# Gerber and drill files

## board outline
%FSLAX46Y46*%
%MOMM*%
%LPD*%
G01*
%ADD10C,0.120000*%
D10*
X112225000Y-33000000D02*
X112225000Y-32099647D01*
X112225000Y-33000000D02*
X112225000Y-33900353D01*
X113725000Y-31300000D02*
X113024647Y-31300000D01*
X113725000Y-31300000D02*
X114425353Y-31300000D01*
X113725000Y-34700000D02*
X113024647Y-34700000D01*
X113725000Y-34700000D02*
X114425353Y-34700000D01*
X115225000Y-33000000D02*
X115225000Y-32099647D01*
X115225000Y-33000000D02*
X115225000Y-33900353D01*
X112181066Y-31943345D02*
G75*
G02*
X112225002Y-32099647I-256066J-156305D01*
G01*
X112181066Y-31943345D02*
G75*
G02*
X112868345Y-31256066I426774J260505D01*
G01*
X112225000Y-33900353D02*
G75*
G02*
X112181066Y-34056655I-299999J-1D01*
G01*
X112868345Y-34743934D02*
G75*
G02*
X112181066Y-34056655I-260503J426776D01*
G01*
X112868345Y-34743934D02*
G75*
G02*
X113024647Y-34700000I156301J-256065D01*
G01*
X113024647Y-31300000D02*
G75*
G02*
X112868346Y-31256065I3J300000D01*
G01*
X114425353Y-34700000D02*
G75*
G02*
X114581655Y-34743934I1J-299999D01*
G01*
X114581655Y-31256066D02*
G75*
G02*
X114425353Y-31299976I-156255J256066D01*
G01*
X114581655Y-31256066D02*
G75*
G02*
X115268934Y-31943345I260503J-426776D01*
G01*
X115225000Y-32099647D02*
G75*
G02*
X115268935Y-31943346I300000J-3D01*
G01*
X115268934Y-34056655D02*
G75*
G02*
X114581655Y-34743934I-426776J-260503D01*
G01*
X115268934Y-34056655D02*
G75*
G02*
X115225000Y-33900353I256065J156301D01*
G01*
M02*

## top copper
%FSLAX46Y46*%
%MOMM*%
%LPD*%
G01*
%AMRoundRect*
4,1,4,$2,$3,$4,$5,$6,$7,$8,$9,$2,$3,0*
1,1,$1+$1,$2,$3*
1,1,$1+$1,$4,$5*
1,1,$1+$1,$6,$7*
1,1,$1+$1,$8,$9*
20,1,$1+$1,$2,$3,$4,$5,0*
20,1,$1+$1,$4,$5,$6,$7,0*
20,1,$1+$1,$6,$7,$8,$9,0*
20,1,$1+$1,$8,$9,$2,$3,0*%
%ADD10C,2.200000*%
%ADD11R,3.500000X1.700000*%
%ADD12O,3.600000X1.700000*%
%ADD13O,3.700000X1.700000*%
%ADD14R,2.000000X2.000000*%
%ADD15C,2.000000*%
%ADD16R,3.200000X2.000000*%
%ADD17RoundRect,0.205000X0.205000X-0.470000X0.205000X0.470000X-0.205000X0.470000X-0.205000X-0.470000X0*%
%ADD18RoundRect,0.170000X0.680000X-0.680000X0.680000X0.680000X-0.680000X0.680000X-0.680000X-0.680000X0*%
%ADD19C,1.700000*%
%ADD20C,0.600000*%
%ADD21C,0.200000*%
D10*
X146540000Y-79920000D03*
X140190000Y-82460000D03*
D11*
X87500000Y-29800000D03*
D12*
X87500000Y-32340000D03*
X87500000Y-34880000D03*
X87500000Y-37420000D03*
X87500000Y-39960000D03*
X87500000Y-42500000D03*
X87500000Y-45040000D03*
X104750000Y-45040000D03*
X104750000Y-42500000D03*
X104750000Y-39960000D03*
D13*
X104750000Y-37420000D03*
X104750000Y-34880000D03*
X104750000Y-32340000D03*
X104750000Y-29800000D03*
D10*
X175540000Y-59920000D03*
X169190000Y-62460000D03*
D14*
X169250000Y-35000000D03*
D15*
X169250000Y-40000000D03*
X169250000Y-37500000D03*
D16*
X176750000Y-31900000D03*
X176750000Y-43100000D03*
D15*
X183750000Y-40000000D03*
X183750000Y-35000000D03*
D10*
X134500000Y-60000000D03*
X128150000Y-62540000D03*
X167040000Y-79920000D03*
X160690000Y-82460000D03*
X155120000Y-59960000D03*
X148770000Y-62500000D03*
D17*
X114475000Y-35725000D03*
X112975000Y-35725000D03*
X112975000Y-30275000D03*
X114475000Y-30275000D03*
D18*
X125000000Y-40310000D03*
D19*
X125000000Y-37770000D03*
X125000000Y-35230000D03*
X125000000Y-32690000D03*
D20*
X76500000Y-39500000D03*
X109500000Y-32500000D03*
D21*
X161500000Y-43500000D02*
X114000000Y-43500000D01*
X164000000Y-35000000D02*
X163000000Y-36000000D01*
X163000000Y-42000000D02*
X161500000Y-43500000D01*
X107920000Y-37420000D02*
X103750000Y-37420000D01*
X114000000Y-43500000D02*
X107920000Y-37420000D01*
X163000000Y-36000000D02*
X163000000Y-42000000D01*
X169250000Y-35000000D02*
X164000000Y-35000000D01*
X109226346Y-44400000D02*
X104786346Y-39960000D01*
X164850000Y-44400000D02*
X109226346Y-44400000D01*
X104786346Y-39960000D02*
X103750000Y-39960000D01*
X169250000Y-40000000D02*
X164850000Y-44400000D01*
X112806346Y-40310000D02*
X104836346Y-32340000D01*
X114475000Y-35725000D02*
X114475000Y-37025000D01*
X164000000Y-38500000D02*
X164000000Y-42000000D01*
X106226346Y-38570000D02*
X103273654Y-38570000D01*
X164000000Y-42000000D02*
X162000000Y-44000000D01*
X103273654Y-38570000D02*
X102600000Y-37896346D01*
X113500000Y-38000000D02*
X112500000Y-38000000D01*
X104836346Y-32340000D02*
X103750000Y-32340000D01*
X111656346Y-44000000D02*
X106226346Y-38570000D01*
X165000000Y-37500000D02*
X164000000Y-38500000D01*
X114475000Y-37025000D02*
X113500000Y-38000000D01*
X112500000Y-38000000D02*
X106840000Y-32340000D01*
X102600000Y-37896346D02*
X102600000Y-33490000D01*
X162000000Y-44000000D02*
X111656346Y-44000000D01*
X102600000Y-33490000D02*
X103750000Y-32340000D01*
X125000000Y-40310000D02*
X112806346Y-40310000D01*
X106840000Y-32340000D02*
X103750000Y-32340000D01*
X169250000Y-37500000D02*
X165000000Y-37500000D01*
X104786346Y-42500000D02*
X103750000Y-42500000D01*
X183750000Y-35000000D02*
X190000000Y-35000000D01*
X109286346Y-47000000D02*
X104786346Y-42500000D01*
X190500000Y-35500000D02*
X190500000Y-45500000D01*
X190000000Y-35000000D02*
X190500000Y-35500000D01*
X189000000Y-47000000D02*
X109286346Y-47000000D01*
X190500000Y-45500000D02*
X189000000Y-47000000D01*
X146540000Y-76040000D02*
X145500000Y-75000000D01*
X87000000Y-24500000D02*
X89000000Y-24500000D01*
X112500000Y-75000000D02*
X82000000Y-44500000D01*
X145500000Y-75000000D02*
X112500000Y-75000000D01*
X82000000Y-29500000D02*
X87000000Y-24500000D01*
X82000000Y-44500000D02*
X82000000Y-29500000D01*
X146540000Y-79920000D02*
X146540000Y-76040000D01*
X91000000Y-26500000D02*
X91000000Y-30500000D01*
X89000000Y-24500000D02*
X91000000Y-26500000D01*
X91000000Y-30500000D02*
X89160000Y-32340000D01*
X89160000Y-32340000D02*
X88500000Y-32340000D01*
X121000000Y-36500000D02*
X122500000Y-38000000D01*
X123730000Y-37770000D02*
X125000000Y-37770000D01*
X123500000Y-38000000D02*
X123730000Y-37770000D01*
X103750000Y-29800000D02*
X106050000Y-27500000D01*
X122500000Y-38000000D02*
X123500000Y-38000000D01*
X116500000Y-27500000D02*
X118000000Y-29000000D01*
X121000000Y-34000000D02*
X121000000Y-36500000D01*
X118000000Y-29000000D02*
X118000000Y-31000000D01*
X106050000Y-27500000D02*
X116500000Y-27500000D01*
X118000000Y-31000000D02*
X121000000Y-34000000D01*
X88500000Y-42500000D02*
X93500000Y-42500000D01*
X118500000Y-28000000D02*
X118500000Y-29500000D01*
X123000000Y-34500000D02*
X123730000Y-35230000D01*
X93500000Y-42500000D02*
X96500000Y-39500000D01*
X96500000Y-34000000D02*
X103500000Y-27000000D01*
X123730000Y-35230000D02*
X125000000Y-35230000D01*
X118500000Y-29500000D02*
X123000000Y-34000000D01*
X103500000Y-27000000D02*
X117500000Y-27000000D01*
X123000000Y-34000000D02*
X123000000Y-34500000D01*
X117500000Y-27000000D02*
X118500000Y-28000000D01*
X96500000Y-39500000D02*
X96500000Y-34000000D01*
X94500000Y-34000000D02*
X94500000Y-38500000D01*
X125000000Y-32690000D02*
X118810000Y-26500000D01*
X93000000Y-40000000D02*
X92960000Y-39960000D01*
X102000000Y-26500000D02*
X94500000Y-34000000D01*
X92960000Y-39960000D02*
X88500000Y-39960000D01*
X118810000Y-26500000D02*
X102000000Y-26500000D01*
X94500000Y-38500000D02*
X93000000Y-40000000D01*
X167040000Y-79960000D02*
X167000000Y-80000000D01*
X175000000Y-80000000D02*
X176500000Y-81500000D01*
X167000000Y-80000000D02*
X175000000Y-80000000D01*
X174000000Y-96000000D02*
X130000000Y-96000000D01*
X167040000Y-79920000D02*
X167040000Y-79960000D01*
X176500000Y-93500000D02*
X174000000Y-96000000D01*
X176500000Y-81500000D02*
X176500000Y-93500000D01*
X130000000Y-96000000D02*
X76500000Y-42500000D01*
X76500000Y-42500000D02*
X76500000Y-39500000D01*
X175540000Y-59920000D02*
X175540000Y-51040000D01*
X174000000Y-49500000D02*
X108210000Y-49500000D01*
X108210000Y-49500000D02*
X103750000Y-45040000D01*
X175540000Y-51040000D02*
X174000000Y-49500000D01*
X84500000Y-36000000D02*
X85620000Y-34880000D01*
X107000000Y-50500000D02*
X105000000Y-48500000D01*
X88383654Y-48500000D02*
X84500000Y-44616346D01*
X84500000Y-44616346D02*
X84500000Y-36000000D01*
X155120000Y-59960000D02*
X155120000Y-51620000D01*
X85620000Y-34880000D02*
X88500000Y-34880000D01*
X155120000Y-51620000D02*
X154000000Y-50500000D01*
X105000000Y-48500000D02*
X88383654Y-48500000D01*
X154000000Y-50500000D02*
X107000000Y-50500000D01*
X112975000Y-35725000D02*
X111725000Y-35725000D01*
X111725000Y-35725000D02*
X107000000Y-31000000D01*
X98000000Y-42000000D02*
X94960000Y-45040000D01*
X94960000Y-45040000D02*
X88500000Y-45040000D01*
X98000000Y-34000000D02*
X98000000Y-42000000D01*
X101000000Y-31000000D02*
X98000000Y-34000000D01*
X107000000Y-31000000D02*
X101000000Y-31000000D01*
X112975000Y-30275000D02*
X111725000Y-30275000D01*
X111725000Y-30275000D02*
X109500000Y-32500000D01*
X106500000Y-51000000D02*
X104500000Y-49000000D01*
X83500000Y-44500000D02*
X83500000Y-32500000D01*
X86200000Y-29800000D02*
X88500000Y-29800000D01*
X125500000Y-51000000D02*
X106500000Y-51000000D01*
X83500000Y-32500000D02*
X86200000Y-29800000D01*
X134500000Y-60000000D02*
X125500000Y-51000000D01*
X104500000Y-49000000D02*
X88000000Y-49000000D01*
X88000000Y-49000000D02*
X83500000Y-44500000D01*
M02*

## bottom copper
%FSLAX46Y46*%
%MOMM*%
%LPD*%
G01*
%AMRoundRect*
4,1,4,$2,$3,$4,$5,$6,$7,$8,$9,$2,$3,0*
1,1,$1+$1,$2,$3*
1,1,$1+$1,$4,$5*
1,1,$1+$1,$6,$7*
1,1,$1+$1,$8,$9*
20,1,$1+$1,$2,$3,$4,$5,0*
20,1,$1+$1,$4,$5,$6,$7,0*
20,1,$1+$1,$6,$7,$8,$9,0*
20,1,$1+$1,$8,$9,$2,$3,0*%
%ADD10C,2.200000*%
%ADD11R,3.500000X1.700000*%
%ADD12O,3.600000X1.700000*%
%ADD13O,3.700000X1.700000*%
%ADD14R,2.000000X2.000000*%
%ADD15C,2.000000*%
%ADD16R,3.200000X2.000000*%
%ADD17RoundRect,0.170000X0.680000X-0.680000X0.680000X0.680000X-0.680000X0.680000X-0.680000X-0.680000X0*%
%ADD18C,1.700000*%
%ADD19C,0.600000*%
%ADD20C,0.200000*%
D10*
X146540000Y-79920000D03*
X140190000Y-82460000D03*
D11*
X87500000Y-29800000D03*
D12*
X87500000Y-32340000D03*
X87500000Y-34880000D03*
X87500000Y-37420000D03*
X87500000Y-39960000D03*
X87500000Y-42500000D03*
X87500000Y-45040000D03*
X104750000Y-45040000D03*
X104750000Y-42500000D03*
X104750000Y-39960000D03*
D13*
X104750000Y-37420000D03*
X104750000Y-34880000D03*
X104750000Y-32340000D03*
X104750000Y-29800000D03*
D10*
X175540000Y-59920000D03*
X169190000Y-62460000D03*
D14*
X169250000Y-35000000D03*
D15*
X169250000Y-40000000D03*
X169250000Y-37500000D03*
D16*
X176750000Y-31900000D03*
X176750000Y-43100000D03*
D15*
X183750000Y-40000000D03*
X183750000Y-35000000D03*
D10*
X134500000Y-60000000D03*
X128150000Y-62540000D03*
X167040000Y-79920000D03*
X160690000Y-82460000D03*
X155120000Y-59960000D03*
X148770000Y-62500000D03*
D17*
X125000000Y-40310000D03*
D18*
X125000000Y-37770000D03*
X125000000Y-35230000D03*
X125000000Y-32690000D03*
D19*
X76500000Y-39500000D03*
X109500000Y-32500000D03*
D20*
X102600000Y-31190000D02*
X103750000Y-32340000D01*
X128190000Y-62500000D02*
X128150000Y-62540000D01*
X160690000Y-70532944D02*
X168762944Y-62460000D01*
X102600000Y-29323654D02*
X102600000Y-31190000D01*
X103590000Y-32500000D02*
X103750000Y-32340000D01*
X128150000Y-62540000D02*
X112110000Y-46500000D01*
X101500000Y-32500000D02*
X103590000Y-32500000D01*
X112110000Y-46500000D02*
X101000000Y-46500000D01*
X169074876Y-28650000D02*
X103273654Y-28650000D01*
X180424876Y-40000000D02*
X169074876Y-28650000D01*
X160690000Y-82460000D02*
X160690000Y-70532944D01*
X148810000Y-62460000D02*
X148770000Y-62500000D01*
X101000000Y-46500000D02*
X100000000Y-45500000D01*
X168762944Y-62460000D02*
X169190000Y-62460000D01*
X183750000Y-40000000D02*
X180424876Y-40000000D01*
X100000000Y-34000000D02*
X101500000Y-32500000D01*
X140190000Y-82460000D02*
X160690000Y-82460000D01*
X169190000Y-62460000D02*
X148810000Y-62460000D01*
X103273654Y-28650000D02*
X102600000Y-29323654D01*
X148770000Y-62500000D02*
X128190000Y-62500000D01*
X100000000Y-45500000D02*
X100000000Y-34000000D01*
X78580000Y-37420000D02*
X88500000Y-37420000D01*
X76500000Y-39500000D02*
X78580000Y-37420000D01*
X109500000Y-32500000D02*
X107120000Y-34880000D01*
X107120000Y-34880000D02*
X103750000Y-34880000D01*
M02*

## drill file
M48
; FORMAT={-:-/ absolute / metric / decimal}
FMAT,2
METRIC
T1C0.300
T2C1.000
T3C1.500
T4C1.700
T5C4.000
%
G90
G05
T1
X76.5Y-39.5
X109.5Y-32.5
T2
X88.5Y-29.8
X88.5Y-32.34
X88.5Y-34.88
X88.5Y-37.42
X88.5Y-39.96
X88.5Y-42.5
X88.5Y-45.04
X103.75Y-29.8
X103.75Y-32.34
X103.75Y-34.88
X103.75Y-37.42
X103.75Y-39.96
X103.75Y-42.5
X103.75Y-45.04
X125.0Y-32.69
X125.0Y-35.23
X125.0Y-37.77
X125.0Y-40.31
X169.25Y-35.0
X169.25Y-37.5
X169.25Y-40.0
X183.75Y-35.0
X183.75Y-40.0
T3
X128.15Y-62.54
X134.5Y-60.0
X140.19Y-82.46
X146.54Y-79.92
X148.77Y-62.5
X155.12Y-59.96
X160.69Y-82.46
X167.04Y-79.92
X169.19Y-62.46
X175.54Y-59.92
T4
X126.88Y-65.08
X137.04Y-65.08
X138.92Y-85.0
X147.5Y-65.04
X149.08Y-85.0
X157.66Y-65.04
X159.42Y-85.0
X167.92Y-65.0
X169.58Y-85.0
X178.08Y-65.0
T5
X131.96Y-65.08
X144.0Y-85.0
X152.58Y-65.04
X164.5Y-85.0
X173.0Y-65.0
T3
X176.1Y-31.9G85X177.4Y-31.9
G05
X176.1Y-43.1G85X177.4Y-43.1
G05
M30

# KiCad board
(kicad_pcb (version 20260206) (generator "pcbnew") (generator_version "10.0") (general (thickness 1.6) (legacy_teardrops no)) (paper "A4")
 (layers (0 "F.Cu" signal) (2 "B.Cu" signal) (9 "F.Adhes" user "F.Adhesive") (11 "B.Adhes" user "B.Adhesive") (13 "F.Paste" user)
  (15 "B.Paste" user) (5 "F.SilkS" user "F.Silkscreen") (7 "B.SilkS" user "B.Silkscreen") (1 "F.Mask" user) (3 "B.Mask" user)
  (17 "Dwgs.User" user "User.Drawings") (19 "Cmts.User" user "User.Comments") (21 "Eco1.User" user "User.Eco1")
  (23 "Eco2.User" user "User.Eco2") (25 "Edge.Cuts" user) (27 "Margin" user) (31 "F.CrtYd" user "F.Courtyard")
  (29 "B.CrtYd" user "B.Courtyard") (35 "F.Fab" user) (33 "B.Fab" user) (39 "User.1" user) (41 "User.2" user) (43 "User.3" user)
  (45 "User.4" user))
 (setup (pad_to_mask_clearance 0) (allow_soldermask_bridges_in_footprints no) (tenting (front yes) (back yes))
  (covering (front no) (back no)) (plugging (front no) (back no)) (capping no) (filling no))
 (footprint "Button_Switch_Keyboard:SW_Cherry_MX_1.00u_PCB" (layer "F.Cu") (at 146.54 79.92)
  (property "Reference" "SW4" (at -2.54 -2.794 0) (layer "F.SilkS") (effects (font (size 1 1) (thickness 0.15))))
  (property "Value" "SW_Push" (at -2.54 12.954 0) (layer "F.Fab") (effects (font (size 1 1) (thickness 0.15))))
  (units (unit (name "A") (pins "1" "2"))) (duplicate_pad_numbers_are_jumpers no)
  (pad "" np_thru_hole circle (at -7.62 5.08) (size 1.7 1.7) (drill 1.7) (layers "*.Cu" "*.Mask"))
  (pad "" np_thru_hole circle (at -2.54 5.08) (size 4 4) (drill 4) (layers "*.Cu" "*.Mask"))
  (pad "" np_thru_hole circle (at 2.54 5.08) (size 1.7 1.7) (drill 1.7) (layers "*.Cu" "*.Mask"))
  (pad "1" thru_hole circle (at 0 0) (size 2.2 2.2) (drill 1.5) (layers "*.Cu" "*.Mask") (remove_unused_layers no)
   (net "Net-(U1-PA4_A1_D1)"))
  (pad "2" thru_hole circle (at -6.35 2.54) (size 2.2 2.2) (drill 1.5) (layers "*.Cu" "*.Mask") (remove_unused_layers no) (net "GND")))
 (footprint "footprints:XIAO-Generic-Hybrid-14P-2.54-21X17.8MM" (layer "F.Cu") (at 96.125 37.42)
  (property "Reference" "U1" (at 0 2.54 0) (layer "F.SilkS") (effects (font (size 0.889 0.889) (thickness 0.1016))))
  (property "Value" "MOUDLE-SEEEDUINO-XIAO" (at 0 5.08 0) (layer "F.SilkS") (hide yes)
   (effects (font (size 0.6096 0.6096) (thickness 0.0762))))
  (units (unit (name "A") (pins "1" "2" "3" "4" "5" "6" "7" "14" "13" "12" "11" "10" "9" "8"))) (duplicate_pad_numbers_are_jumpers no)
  (pad "1" thru_hole rect (at -7.625 -7.62) (size 3.5 1.7) (drill 1 (offset -1 0)) (layers "*.Cu" "*.Mask") (remove_unused_layers no)
   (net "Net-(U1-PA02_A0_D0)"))
  (pad "2" thru_hole oval (at -7.625 -5.08) (size 3.6 1.7) (drill 1 (offset -1 0)) (layers "*.Cu" "*.Mask") (remove_unused_layers no)
   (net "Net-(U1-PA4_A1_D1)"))
  (pad "3" thru_hole oval (at -7.625 -2.54) (size 3.6 1.7) (drill 1 (offset -1 0)) (layers "*.Cu" "*.Mask") (remove_unused_layers no)
   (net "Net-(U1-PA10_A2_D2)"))
  (pad "4" thru_hole oval (at -7.625 0) (size 3.6 1.7) (drill 1 (offset -1 0)) (layers "*.Cu" "*.Mask") (remove_unused_layers no)
   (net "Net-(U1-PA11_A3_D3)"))
  (pad "5" thru_hole oval (at -7.625 2.54) (size 3.6 1.7) (drill 1 (offset -1 0)) (layers "*.Cu" "*.Mask") (remove_unused_layers no)
   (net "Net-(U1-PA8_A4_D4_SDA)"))
  (pad "6" thru_hole oval (at -7.625 5.08 180) (size 3.6 1.7) (drill 1 (offset 1 0)) (layers "*.Cu" "*.Mask") (remove_unused_layers no)
   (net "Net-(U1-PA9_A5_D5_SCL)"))
  (pad "7" thru_hole oval (at -7.625 7.62) (size 3.6 1.7) (drill 1 (offset -1 0)) (layers "*.Cu" "*.Mask") (remove_unused_layers no)
   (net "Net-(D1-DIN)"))
  (pad "8" thru_hole oval (at 7.625 7.62) (size 3.6 1.7) (drill 1 (offset 1 0)) (layers "*.Cu" "*.Mask") (remove_unused_layers no)
   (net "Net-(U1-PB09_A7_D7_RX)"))
  (pad "9" thru_hole oval (at 7.625 5.08) (size 3.6 1.7) (drill 1 (offset 1 0)) (layers "*.Cu" "*.Mask") (remove_unused_layers no)
   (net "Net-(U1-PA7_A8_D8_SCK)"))
  (pad "10" thru_hole oval (at 7.625 2.54) (size 3.6 1.7) (drill 1 (offset 1 0)) (layers "*.Cu" "*.Mask") (remove_unused_layers no)
   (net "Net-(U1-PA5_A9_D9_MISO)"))
  (pad "11" thru_hole oval (at 7.625 0) (size 3.7 1.7) (drill 1 (offset 1 0)) (layers "*.Cu" "*.Mask") (remove_unused_layers no)
   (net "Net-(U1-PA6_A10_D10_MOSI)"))
  (pad "12" thru_hole oval (at 7.625 -2.54) (size 3.7 1.7) (drill 1 (offset 1 0)) (layers "*.Cu" "*.Mask") (remove_unused_layers no)
   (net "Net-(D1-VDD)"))
  (pad "13" thru_hole oval (at 7.625 -5.08) (size 3.7 1.7) (drill 1 (offset 1 0)) (layers "*.Cu" "*.Mask") (remove_unused_layers no)
   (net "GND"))
  (pad "14" thru_hole oval (at 7.625 -7.62) (size 3.7 1.7) (drill 1 (offset 1 0)) (layers "*.Cu" "*.Mask") (remove_unused_layers no)
   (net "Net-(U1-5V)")))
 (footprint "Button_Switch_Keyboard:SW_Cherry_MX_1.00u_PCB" (layer "F.Cu") (at 175.54 59.92)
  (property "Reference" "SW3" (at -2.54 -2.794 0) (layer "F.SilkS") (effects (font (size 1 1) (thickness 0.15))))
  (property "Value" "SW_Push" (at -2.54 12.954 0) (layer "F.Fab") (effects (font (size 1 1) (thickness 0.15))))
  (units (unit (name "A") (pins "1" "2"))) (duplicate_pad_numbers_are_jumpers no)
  (pad "" np_thru_hole circle (at -7.62 5.08) (size 1.7 1.7) (drill 1.7) (layers "*.Cu" "*.Mask"))
  (pad "" np_thru_hole circle (at -2.54 5.08) (size 4 4) (drill 4) (layers "*.Cu" "*.Mask"))
  (pad "" np_thru_hole circle (at 2.54 5.08) (size 1.7 1.7) (drill 1.7) (layers "*.Cu" "*.Mask"))
  (pad "1" thru_hole circle (at 0 0) (size 2.2 2.2) (drill 1.5) (layers "*.Cu" "*.Mask") (remove_unused_layers no)
   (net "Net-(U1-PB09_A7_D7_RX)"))
  (pad "2" thru_hole circle (at -6.35 2.54) (size 2.2 2.2) (drill 1.5) (layers "*.Cu" "*.Mask") (remove_unused_layers no) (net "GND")))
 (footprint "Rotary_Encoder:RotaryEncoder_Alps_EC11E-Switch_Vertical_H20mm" (layer "F.Cu") (at 169.25 35)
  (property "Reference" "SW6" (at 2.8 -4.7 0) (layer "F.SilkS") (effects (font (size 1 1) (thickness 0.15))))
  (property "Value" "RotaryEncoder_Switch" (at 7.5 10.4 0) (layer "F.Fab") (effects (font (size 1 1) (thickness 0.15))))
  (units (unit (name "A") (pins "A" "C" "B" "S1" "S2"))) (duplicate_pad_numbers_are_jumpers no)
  (pad "A" thru_hole rect (at 0 0) (size 2 2) (drill 1) (layers "*.Cu" "*.Mask") (remove_unused_layers no) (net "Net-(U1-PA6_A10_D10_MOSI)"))
  (pad "B" thru_hole circle (at 0 5) (size 2 2) (drill 1) (layers "*.Cu" "*.Mask") (remove_unused_layers no) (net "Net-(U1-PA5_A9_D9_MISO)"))
  (pad "C" thru_hole circle (at 0 2.5) (size 2 2) (drill 1) (layers "*.Cu" "*.Mask") (remove_unused_layers no) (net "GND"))
  (pad "MP" thru_hole rect (at 7.5 -3.1) (size 3.2 2) (drill oval 2.8 1.5) (layers "*.Cu" "*.Mask") (remove_unused_layers no))
  (pad "MP" thru_hole rect (at 7.5 8.1) (size 3.2 2) (drill oval 2.8 1.5) (layers "*.Cu" "*.Mask") (remove_unused_layers no))
  (pad "S1" thru_hole circle (at 14.5 5) (size 2 2) (drill 1) (layers "*.Cu" "*.Mask") (remove_unused_layers no) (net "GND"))
  (pad "S2" thru_hole circle (at 14.5 0) (size 2 2) (drill 1) (layers "*.Cu" "*.Mask") (remove_unused_layers no)
   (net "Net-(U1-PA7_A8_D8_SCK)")))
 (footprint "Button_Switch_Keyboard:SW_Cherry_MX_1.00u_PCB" (layer "F.Cu") (at 134.5 60)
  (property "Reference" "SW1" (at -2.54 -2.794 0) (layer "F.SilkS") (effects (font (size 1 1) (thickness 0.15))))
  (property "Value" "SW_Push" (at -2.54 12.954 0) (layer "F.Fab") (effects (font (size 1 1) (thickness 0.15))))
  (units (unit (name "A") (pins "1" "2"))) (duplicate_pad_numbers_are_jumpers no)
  (pad "" np_thru_hole circle (at -7.62 5.08) (size 1.7 1.7) (drill 1.7) (layers "*.Cu" "*.Mask"))
  (pad "" np_thru_hole circle (at -2.54 5.08) (size 4 4) (drill 4) (layers "*.Cu" "*.Mask"))
  (pad "" np_thru_hole circle (at 2.54 5.08) (size 1.7 1.7) (drill 1.7) (layers "*.Cu" "*.Mask"))
  (pad "1" thru_hole circle (at 0 0) (size 2.2 2.2) (drill 1.5) (layers "*.Cu" "*.Mask") (remove_unused_layers no)
   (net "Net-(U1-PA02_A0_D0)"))
  (pad "2" thru_hole circle (at -6.35 2.54) (size 2.2 2.2) (drill 1.5) (layers "*.Cu" "*.Mask") (remove_unused_layers no) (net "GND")))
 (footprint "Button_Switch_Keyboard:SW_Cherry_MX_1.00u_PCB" (layer "F.Cu") (at 167.04 79.92)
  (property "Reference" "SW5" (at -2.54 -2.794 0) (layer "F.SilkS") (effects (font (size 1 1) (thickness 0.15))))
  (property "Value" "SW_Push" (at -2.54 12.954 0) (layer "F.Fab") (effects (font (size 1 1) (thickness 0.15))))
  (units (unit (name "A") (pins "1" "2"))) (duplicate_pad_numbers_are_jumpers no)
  (pad "" np_thru_hole circle (at -7.62 5.08) (size 1.7 1.7) (drill 1.7) (layers "*.Cu" "*.Mask"))
  (pad "" np_thru_hole circle (at -2.54 5.08) (size 4 4) (drill 4) (layers "*.Cu" "*.Mask"))
  (pad "" np_thru_hole circle (at 2.54 5.08) (size 1.7 1.7) (drill 1.7) (layers "*.Cu" "*.Mask"))
  (pad "1" thru_hole circle (at 0 0) (size 2.2 2.2) (drill 1.5) (layers "*.Cu" "*.Mask") (remove_unused_layers no)
   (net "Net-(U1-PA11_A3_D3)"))
  (pad "2" thru_hole circle (at -6.35 2.54) (size 2.2 2.2) (drill 1.5) (layers "*.Cu" "*.Mask") (remove_unused_layers no) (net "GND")))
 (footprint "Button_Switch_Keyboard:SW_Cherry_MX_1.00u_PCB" (layer "F.Cu") (at 155.12 59.96)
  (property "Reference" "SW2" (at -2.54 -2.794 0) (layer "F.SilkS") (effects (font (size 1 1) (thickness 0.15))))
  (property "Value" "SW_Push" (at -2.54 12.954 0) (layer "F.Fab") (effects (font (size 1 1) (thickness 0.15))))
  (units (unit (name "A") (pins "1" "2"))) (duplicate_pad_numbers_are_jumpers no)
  (pad "" np_thru_hole circle (at -7.62 5.08) (size 1.7 1.7) (drill 1.7) (layers "*.Cu" "*.Mask"))
  (pad "" np_thru_hole circle (at -2.54 5.08) (size 4 4) (drill 4) (layers "*.Cu" "*.Mask"))
  (pad "" np_thru_hole circle (at 2.54 5.08) (size 1.7 1.7) (drill 1.7) (layers "*.Cu" "*.Mask"))
  (pad "1" thru_hole circle (at 0 0) (size 2.2 2.2) (drill 1.5) (layers "*.Cu" "*.Mask") (remove_unused_layers no)
   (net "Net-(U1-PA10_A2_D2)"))
  (pad "2" thru_hole circle (at -6.35 2.54) (size 2.2 2.2) (drill 1.5) (layers "*.Cu" "*.Mask") (remove_unused_layers no) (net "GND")))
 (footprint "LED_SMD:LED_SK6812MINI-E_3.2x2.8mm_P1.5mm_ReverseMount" (layer "F.Cu") (at 113.725 33 90)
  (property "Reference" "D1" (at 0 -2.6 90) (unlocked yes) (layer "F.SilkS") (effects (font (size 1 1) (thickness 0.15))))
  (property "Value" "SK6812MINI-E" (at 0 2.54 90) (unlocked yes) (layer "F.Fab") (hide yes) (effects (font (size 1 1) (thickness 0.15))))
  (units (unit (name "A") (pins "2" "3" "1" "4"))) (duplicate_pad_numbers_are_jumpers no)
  (fp_line (start 0 -1.5) (end 0.900353 -1.5) (stroke (width 0.12) (type solid)) (layer "Edge.Cuts"))
  (fp_line (start 0 -1.5) (end -0.900353 -1.5) (stroke (width 0.12) (type solid)) (layer "Edge.Cuts"))
  (fp_line (start 1.7 0) (end 1.7 -0.700353) (stroke (width 0.12) (type solid)) (layer "Edge.Cuts"))
  (fp_line (start 1.7 0) (end 1.7 0.700353) (stroke (width 0.12) (type solid)) (layer "Edge.Cuts"))
  (fp_line (start -1.7 0) (end -1.7 -0.700353) (stroke (width 0.12) (type solid)) (layer "Edge.Cuts"))
  (fp_line (start -1.7 0) (end -1.7 0.700353) (stroke (width 0.12) (type solid)) (layer "Edge.Cuts"))
  (fp_line (start 0 1.5) (end 0.900353 1.5) (stroke (width 0.12) (type solid)) (layer "Edge.Cuts"))
  (fp_line (start 0 1.5) (end -0.900353 1.5) (stroke (width 0.12) (type solid)) (layer "Edge.Cuts"))
  (fp_arc (start 1.056655 -1.543934) (mid 0.981532 -1.511192) (end 0.900353 -1.5) (stroke (width 0.12) (type solid)) (layer "Edge.Cuts"))
  (fp_arc (start 1.056655 -1.543934) (mid 1.670711 -1.470711) (end 1.743934 -0.856655) (stroke (width 0.12) (type solid))
   (layer "Edge.Cuts"))
  (fp_arc (start -0.900353 -1.5) (mid -0.981532 -1.511192) (end -1.056655 -1.543934) (stroke (width 0.12) (type solid)) (layer "Edge.Cuts"))
  (fp_arc (start -1.743934 -0.856655) (mid -1.670711 -1.470711) (end -1.056655 -1.543934) (stroke (width 0.12) (type solid))
   (layer "Edge.Cuts"))
  (fp_arc (start -1.743934 -0.856655) (mid -1.711192 -0.781532) (end -1.7 -0.700353) (stroke (width 0.12) (type solid)) (layer "Edge.Cuts"))
  (fp_arc (start 1.7 -0.700353) (mid 1.711192 -0.781532) (end 1.743934 -0.856655) (stroke (width 0.12) (type solid)) (layer "Edge.Cuts"))
  (fp_arc (start -1.7 0.700353) (mid -1.711192 0.781532) (end -1.743934 0.856655) (stroke (width 0.12) (type solid)) (layer "Edge.Cuts"))
  (fp_arc (start 1.743934 0.856655) (mid 1.711192 0.781532) (end 1.7 0.700353) (stroke (width 0.12) (type solid)) (layer "Edge.Cuts"))
  (fp_arc (start 1.743934 0.856655) (mid 1.670711 1.470711) (end 1.056655 1.543934) (stroke (width 0.12) (type solid)) (layer "Edge.Cuts"))
  (fp_arc (start 0.900353 1.5) (mid 0.981532 1.511192) (end 1.056655 1.543934) (stroke (width 0.12) (type solid)) (layer "Edge.Cuts"))
  (fp_arc (start -1.056655 1.543934) (mid -1.670711 1.470711) (end -1.743934 0.856655) (stroke (width 0.12) (type solid))
   (layer "Edge.Cuts"))
  (fp_arc (start -1.056655 1.543934) (mid -0.981532 1.511192) (end -0.900353 1.5) (stroke (width 0.12) (type solid)) (layer "Edge.Cuts"))
  (pad "1" smd roundrect (at -2.725 0.75 90) (size 1.35 0.82) (layers "F.Cu" "F.Mask" "F.Paste") (roundrect_rratio 0.25) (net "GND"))
  (pad "2" smd roundrect (at -2.725 -0.75 90) (size 1.35 0.82) (layers "F.Cu" "F.Mask" "F.Paste") (roundrect_rratio 0.25)
   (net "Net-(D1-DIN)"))
  (pad "3" smd roundrect (at 2.725 -0.75 90) (size 1.35 0.82) (layers "F.Cu" "F.Mask" "F.Paste") (roundrect_rratio 0.25)
   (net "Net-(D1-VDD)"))
  (pad "4" smd roundrect (at 2.725 0.75 90) (size 1.35 0.82) (layers "F.Cu" "F.Mask" "F.Paste") (roundrect_rratio 0.25)
   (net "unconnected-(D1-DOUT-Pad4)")))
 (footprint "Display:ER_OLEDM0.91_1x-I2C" (layer "F.Cu") (at 125 40.31 90)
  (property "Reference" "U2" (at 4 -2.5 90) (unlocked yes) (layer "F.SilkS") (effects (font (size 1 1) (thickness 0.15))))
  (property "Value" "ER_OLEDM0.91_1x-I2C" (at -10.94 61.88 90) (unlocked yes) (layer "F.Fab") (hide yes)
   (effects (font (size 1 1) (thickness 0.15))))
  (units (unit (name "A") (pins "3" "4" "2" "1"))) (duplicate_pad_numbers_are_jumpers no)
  (pad "1" thru_hole roundrect (at 0 0 90) (size 1.7 1.7) (drill 1) (layers "*.Cu" "*.Mask") (remove_unused_layers no)
   (roundrect_rratio 0.1) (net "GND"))
  (pad "2" thru_hole circle (at 2.54 0 90) (size 1.7 1.7) (drill 1) (layers "*.Cu" "*.Mask") (remove_unused_layers no) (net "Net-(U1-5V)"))
  (pad "3" thru_hole circle (at 5.08 0 90) (size 1.7 1.7) (drill 1) (layers "*.Cu" "*.Mask") (remove_unused_layers no)
   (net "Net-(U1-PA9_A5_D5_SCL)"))
  (pad "4" thru_hole circle (at 7.62 0 90) (size 1.7 1.7) (drill 1) (layers "*.Cu" "*.Mask") (remove_unused_layers no)
   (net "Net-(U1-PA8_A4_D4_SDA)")))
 (segment (start 161.5 43.5) (end 114 43.5) (width 0.2) (layer "F.Cu") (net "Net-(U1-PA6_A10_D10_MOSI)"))
 (segment (start 164 35) (end 163 36) (width 0.2) (layer "F.Cu") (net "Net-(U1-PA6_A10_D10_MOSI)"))
 (segment (start 163 42) (end 161.5 43.5) (width 0.2) (layer "F.Cu") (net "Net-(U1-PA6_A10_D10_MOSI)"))
 (segment (start 107.92 37.42) (end 103.75 37.42) (width 0.2) (layer "F.Cu") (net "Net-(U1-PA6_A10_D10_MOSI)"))
 (segment (start 114 43.5) (end 107.92 37.42) (width 0.2) (layer "F.Cu") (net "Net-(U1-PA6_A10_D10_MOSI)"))
 (segment (start 163 36) (end 163 42) (width 0.2) (layer "F.Cu") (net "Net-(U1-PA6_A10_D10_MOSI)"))
 (segment (start 169.25 35) (end 164 35) (width 0.2) (layer "F.Cu") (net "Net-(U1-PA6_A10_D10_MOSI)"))
 (segment (start 109.226346 44.4) (end 104.786346 39.96) (width 0.2) (layer "F.Cu") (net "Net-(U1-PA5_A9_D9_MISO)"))
 (segment (start 164.85 44.4) (end 109.226346 44.4) (width 0.2) (layer "F.Cu") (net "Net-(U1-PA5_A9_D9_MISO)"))
 (segment (start 104.786346 39.96) (end 103.75 39.96) (width 0.2) (layer "F.Cu") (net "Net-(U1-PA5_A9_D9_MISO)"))
 (segment (start 169.25 40) (end 164.85 44.4) (width 0.2) (layer "F.Cu") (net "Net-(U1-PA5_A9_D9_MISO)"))
 (segment (start 112.806346 40.31) (end 104.836346 32.34) (width 0.2) (layer "F.Cu") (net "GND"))
 (segment (start 114.475 35.725) (end 114.475 37.025) (width 0.2) (layer "F.Cu") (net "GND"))
 (segment (start 164 38.5) (end 164 42) (width 0.2) (layer "F.Cu") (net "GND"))
 (segment (start 106.226346 38.57) (end 103.273654 38.57) (width 0.2) (layer "F.Cu") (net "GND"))
 (segment (start 164 42) (end 162 44) (width 0.2) (layer "F.Cu") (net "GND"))
 (segment (start 103.273654 38.57) (end 102.6 37.896346) (width 0.2) (layer "F.Cu") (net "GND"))
 (segment (start 113.5 38) (end 112.5 38) (width 0.2) (layer "F.Cu") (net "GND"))
 (segment (start 104.836346 32.34) (end 103.75 32.34) (width 0.2) (layer "F.Cu") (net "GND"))
 (segment (start 111.656346 44) (end 106.226346 38.57) (width 0.2) (layer "F.Cu") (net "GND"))
 (segment (start 165 37.5) (end 164 38.5) (width 0.2) (layer "F.Cu") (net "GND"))
 (segment (start 114.475 37.025) (end 113.5 38) (width 0.2) (layer "F.Cu") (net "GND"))
 (segment (start 112.5 38) (end 106.84 32.34) (width 0.2) (layer "F.Cu") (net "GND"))
 (segment (start 102.6 37.896346) (end 102.6 33.49) (width 0.2) (layer "F.Cu") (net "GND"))
 (segment (start 162 44) (end 111.656346 44) (width 0.2) (layer "F.Cu") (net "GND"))
 (segment (start 102.6 33.49) (end 103.75 32.34) (width 0.2) (layer "F.Cu") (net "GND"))
 (segment (start 125 40.31) (end 112.806346 40.31) (width 0.2) (layer "F.Cu") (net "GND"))
 (segment (start 106.84 32.34) (end 103.75 32.34) (width 0.2) (layer "F.Cu") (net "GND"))
 (segment (start 169.25 37.5) (end 165 37.5) (width 0.2) (layer "F.Cu") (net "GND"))
 (segment (start 102.6 31.19) (end 103.75 32.34) (width 0.2) (layer "B.Cu") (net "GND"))
 (segment (start 128.19 62.5) (end 128.15 62.54) (width 0.2) (layer "B.Cu") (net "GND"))
 (segment (start 160.69 70.532944) (end 168.762944 62.46) (width 0.2) (layer "B.Cu") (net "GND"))
 (segment (start 102.6 29.323654) (end 102.6 31.19) (width 0.2) (layer "B.Cu") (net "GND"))
 (segment (start 103.59 32.5) (end 103.75 32.34) (width 0.2) (layer "B.Cu") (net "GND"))
 (segment (start 128.15 62.54) (end 112.11 46.5) (width 0.2) (layer "B.Cu") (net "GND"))
 (segment (start 101.5 32.5) (end 103.59 32.5) (width 0.2) (layer "B.Cu") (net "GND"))
 (segment (start 112.11 46.5) (end 101 46.5) (width 0.2) (layer "B.Cu") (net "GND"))
 (segment (start 169.074876 28.65) (end 103.273654 28.65) (width 0.2) (layer "B.Cu") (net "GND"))
 (segment (start 180.424876 40) (end 169.074876 28.65) (width 0.2) (layer "B.Cu") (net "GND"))
 (segment (start 160.69 82.46) (end 160.69 70.532944) (width 0.2) (layer "B.Cu") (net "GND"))
 (segment (start 148.81 62.46) (end 148.77 62.5) (width 0.2) (layer "B.Cu") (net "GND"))
 (segment (start 101 46.5) (end 100 45.5) (width 0.2) (layer "B.Cu") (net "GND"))
 (segment (start 168.762944 62.46) (end 169.19 62.46) (width 0.2) (layer "B.Cu") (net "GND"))
 (segment (start 183.75 40) (end 180.424876 40) (width 0.2) (layer "B.Cu") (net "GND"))
 (segment (start 100 34) (end 101.5 32.5) (width 0.2) (layer "B.Cu") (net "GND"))
 (segment (start 140.19 82.46) (end 160.69 82.46) (width 0.2) (layer "B.Cu") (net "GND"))
 (segment (start 169.19 62.46) (end 148.81 62.46) (width 0.2) (layer "B.Cu") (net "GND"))
 (segment (start 103.273654 28.65) (end 102.6 29.323654) (width 0.2) (layer "B.Cu") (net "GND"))
 (segment (start 148.77 62.5) (end 128.19 62.5) (width 0.2) (layer "B.Cu") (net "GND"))
 (segment (start 100 45.5) (end 100 34) (width 0.2) (layer "B.Cu") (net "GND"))
 (segment (start 104.786346 42.5) (end 103.75 42.5) (width 0.2) (layer "F.Cu") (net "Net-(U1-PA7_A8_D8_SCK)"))
 (segment (start 183.75 35) (end 190 35) (width 0.2) (layer "F.Cu") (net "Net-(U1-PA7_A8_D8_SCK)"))
 (segment (start 109.286346 47) (end 104.786346 42.5) (width 0.2) (layer "F.Cu") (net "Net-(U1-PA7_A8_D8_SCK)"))
 (segment (start 190.5 35.5) (end 190.5 45.5) (width 0.2) (layer "F.Cu") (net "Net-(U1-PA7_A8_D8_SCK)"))
 (segment (start 190 35) (end 190.5 35.5) (width 0.2) (layer "F.Cu") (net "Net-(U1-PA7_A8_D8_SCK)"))
 (segment (start 189 47) (end 109.286346 47) (width 0.2) (layer "F.Cu") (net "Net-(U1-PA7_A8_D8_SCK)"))
 (segment (start 190.5 45.5) (end 189 47) (width 0.2) (layer "F.Cu") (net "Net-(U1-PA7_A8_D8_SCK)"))
 (segment (start 146.54 76.04) (end 145.5 75) (width 0.2) (layer "F.Cu") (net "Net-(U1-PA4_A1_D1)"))
 (segment (start 87 24.5) (end 89 24.5) (width 0.2) (layer "F.Cu") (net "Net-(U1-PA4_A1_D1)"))
 (segment (start 112.5 75) (end 82 44.5) (width 0.2) (layer "F.Cu") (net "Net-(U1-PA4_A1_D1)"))
 (segment (start 145.5 75) (end 112.5 75) (width 0.2) (layer "F.Cu") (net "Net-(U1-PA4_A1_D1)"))
 (segment (start 82 29.5) (end 87 24.5) (width 0.2) (layer "F.Cu") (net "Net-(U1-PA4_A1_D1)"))
 (segment (start 82 44.5) (end 82 29.5) (width 0.2) (layer "F.Cu") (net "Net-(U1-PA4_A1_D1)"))
 (segment (start 146.54 79.92) (end 146.54 76.04) (width 0.2) (layer "F.Cu") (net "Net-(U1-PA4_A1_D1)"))
 (segment (start 91 26.5) (end 91 30.5) (width 0.2) (layer "F.Cu") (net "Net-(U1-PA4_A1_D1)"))
 (segment (start 89 24.5) (end 91 26.5) (width 0.2) (layer "F.Cu") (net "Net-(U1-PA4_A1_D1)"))
 (segment (start 91 30.5) (end 89.16 32.34) (width 0.2) (layer "F.Cu") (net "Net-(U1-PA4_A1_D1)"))
 (segment (start 89.16 32.34) (end 88.5 32.34) (width 0.2) (layer "F.Cu") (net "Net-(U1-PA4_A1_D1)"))
 (segment (start 121 36.5) (end 122.5 38) (width 0.2) (layer "F.Cu") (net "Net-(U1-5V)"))
 (segment (start 123.73 37.77) (end 125 37.77) (width 0.2) (layer "F.Cu") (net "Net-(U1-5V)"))
 (segment (start 123.5 38) (end 123.73 37.77) (width 0.2) (layer "F.Cu") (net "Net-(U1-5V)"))
 (segment (start 103.75 29.8) (end 106.05 27.5) (width 0.2) (layer "F.Cu") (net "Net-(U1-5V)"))
 (segment (start 122.5 38) (end 123.5 38) (width 0.2) (layer "F.Cu") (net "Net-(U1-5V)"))
 (segment (start 116.5 27.5) (end 118 29) (width 0.2) (layer "F.Cu") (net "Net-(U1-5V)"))
 (segment (start 121 34) (end 121 36.5) (width 0.2) (layer "F.Cu") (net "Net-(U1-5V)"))
 (segment (start 118 29) (end 118 31) (width 0.2) (layer "F.Cu") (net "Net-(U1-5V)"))
 (segment (start 106.05 27.5) (end 116.5 27.5) (width 0.2) (layer "F.Cu") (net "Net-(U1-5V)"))
 (segment (start 118 31) (end 121 34) (width 0.2) (layer "F.Cu") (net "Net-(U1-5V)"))
 (segment (start 88.5 42.5) (end 93.5 42.5) (width 0.2) (layer "F.Cu") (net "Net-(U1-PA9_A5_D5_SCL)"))
 (segment (start 118.5 28) (end 118.5 29.5) (width 0.2) (layer "F.Cu") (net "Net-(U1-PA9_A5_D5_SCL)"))
 (segment (start 123 34.5) (end 123.73 35.23) (width 0.2) (layer "F.Cu") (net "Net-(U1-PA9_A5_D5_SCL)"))
 (segment (start 93.5 42.5) (end 96.5 39.5) (width 0.2) (layer "F.Cu") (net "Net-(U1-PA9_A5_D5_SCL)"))
 (segment (start 96.5 34) (end 103.5 27) (width 0.2) (layer "F.Cu") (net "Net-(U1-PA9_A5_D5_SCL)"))
 (segment (start 123.73 35.23) (end 125 35.23) (width 0.2) (layer "F.Cu") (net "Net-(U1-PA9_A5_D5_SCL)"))
 (segment (start 118.5 29.5) (end 123 34) (width 0.2) (layer "F.Cu") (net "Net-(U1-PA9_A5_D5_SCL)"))
 (segment (start 103.5 27) (end 117.5 27) (width 0.2) (layer "F.Cu") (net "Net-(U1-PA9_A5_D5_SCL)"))
 (segment (start 123 34) (end 123 34.5) (width 0.2) (layer "F.Cu") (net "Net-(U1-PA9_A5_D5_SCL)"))
 (segment (start 117.5 27) (end 118.5 28) (width 0.2) (layer "F.Cu") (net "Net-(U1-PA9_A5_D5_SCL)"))
 (segment (start 96.5 39.5) (end 96.5 34) (width 0.2) (layer "F.Cu") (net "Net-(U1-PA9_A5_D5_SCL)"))
 (segment (start 94.5 34) (end 94.5 38.5) (width 0.2) (layer "F.Cu") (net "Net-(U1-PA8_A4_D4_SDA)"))
 (segment (start 125 32.69) (end 118.81 26.5) (width 0.2) (layer "F.Cu") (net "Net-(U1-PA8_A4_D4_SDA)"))
 (segment (start 93 40) (end 92.96 39.96) (width 0.2) (layer "F.Cu") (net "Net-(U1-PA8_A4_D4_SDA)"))
 (segment (start 102 26.5) (end 94.5 34) (width 0.2) (layer "F.Cu") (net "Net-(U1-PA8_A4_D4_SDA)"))
 (segment (start 92.96 39.96) (end 88.5 39.96) (width 0.2) (layer "F.Cu") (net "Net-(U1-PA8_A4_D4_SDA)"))
 (segment (start 118.81 26.5) (end 102 26.5) (width 0.2) (layer "F.Cu") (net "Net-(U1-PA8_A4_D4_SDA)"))
 (segment (start 94.5 38.5) (end 93 40) (width 0.2) (layer "F.Cu") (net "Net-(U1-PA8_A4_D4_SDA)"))
 (segment (start 167.04 79.96) (end 167 80) (width 0.2) (layer "F.Cu") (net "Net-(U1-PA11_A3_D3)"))
 (segment (start 175 80) (end 176.5 81.5) (width 0.2) (layer "F.Cu") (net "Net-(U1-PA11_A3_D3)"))
 (segment (start 167 80) (end 175 80) (width 0.2) (layer "F.Cu") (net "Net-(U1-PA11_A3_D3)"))
 (segment (start 174 96) (end 130 96) (width 0.2) (layer "F.Cu") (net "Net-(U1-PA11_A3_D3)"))
 (segment (start 167.04 79.92) (end 167.04 79.96) (width 0.2) (layer "F.Cu") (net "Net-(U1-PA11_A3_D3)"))
 (segment (start 176.5 93.5) (end 174 96) (width 0.2) (layer "F.Cu") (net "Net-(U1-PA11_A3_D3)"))
 (segment (start 176.5 81.5) (end 176.5 93.5) (width 0.2) (layer "F.Cu") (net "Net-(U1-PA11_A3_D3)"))
 (segment (start 130 96) (end 76.5 42.5) (width 0.2) (layer "F.Cu") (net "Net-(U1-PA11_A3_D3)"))
 (segment (start 76.5 42.5) (end 76.5 39.5) (width 0.2) (layer "F.Cu") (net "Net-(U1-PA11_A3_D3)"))
 (via (at 76.5 39.5) (size 0.6) (drill 0.3) (layers "F.Cu" "B.Cu") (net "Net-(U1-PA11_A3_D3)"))
 (segment (start 78.58 37.42) (end 88.5 37.42) (width 0.2) (layer "B.Cu") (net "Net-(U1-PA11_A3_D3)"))
 (segment (start 76.5 39.5) (end 78.58 37.42) (width 0.2) (layer "B.Cu") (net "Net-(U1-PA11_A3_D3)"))
 (segment (start 175.54 59.92) (end 175.54 51.04) (width 0.2) (layer "F.Cu") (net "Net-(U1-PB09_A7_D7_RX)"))
 (segment (start 174 49.5) (end 108.21 49.5) (width 0.2) (layer "F.Cu") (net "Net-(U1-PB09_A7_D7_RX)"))
 (segment (start 108.21 49.5) (end 103.75 45.04) (width 0.2) (layer "F.Cu") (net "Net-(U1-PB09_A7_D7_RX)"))
 (segment (start 175.54 51.04) (end 174 49.5) (width 0.2) (layer "F.Cu") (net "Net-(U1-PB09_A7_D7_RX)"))
 (segment (start 84.5 36) (end 85.62 34.88) (width 0.2) (layer "F.Cu") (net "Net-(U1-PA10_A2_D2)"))
 (segment (start 107 50.5) (end 105 48.5) (width 0.2) (layer "F.Cu") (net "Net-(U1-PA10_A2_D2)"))
 (segment (start 88.383654 48.5) (end 84.5 44.616346) (width 0.2) (layer "F.Cu") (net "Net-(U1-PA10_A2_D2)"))
 (segment (start 84.5 44.616346) (end 84.5 36) (width 0.2) (layer "F.Cu") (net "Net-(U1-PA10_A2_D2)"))
 (segment (start 155.12 59.96) (end 155.12 51.62) (width 0.2) (layer "F.Cu") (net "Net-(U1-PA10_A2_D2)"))
 (segment (start 85.62 34.88) (end 88.5 34.88) (width 0.2) (layer "F.Cu") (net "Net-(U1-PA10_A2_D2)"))
 (segment (start 155.12 51.62) (end 154 50.5) (width 0.2) (layer "F.Cu") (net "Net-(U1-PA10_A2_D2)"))
 (segment (start 105 48.5) (end 88.383654 48.5) (width 0.2) (layer "F.Cu") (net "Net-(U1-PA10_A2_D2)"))
 (segment (start 154 50.5) (end 107 50.5) (width 0.2) (layer "F.Cu") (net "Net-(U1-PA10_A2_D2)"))
 (segment (start 112.975 35.725) (end 111.725 35.725) (width 0.2) (layer "F.Cu") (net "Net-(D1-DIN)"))
 (segment (start 111.725 35.725) (end 107 31) (width 0.2) (layer "F.Cu") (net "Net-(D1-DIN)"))
 (segment (start 98 42) (end 94.96 45.04) (width 0.2) (layer "F.Cu") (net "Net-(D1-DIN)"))
 (segment (start 94.96 45.04) (end 88.5 45.04) (width 0.2) (layer "F.Cu") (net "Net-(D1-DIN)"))
 (segment (start 98 34) (end 98 42) (width 0.2) (layer "F.Cu") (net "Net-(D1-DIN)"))
 (segment (start 101 31) (end 98 34) (width 0.2) (layer "F.Cu") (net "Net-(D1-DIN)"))
 (segment (start 107 31) (end 101 31) (width 0.2) (layer "F.Cu") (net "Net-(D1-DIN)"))
 (segment (start 112.975 30.275) (end 111.725 30.275) (width 0.2) (layer "F.Cu") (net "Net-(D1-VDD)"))
 (segment (start 111.725 30.275) (end 109.5 32.5) (width 0.2) (layer "F.Cu") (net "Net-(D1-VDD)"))
 (via (at 109.5 32.5) (size 0.6) (drill 0.3) (layers "F.Cu" "B.Cu") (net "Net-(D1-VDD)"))
 (segment (start 109.5 32.5) (end 107.12 34.88) (width 0.2) (layer "B.Cu") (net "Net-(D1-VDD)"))
 (segment (start 107.12 34.88) (end 103.75 34.88) (width 0.2) (layer "B.Cu") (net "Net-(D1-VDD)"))
 (segment (start 106.5 51) (end 104.5 49) (width 0.2) (layer "F.Cu") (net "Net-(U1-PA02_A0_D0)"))
 (segment (start 83.5 44.5) (end 83.5 32.5) (width 0.2) (layer "F.Cu") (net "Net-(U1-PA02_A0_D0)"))
 (segment (start 86.2 29.8) (end 88.5 29.8) (width 0.2) (layer "F.Cu") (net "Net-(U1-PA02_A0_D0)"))
 (segment (start 125.5 51) (end 106.5 51) (width 0.2) (layer "F.Cu") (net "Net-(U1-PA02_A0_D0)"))
 (segment (start 83.5 32.5) (end 86.2 29.8) (width 0.2) (layer "F.Cu") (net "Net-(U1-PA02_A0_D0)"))
 (segment (start 134.5 60) (end 125.5 51) (width 0.2) (layer "F.Cu") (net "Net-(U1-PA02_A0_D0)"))
 (segment (start 104.5 49) (end 88 49) (width 0.2) (layer "F.Cu") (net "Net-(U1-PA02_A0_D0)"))
 (segment (start 88 49) (end 83.5 44.5) (width 0.2) (layer "F.Cu") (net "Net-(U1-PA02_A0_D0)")))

